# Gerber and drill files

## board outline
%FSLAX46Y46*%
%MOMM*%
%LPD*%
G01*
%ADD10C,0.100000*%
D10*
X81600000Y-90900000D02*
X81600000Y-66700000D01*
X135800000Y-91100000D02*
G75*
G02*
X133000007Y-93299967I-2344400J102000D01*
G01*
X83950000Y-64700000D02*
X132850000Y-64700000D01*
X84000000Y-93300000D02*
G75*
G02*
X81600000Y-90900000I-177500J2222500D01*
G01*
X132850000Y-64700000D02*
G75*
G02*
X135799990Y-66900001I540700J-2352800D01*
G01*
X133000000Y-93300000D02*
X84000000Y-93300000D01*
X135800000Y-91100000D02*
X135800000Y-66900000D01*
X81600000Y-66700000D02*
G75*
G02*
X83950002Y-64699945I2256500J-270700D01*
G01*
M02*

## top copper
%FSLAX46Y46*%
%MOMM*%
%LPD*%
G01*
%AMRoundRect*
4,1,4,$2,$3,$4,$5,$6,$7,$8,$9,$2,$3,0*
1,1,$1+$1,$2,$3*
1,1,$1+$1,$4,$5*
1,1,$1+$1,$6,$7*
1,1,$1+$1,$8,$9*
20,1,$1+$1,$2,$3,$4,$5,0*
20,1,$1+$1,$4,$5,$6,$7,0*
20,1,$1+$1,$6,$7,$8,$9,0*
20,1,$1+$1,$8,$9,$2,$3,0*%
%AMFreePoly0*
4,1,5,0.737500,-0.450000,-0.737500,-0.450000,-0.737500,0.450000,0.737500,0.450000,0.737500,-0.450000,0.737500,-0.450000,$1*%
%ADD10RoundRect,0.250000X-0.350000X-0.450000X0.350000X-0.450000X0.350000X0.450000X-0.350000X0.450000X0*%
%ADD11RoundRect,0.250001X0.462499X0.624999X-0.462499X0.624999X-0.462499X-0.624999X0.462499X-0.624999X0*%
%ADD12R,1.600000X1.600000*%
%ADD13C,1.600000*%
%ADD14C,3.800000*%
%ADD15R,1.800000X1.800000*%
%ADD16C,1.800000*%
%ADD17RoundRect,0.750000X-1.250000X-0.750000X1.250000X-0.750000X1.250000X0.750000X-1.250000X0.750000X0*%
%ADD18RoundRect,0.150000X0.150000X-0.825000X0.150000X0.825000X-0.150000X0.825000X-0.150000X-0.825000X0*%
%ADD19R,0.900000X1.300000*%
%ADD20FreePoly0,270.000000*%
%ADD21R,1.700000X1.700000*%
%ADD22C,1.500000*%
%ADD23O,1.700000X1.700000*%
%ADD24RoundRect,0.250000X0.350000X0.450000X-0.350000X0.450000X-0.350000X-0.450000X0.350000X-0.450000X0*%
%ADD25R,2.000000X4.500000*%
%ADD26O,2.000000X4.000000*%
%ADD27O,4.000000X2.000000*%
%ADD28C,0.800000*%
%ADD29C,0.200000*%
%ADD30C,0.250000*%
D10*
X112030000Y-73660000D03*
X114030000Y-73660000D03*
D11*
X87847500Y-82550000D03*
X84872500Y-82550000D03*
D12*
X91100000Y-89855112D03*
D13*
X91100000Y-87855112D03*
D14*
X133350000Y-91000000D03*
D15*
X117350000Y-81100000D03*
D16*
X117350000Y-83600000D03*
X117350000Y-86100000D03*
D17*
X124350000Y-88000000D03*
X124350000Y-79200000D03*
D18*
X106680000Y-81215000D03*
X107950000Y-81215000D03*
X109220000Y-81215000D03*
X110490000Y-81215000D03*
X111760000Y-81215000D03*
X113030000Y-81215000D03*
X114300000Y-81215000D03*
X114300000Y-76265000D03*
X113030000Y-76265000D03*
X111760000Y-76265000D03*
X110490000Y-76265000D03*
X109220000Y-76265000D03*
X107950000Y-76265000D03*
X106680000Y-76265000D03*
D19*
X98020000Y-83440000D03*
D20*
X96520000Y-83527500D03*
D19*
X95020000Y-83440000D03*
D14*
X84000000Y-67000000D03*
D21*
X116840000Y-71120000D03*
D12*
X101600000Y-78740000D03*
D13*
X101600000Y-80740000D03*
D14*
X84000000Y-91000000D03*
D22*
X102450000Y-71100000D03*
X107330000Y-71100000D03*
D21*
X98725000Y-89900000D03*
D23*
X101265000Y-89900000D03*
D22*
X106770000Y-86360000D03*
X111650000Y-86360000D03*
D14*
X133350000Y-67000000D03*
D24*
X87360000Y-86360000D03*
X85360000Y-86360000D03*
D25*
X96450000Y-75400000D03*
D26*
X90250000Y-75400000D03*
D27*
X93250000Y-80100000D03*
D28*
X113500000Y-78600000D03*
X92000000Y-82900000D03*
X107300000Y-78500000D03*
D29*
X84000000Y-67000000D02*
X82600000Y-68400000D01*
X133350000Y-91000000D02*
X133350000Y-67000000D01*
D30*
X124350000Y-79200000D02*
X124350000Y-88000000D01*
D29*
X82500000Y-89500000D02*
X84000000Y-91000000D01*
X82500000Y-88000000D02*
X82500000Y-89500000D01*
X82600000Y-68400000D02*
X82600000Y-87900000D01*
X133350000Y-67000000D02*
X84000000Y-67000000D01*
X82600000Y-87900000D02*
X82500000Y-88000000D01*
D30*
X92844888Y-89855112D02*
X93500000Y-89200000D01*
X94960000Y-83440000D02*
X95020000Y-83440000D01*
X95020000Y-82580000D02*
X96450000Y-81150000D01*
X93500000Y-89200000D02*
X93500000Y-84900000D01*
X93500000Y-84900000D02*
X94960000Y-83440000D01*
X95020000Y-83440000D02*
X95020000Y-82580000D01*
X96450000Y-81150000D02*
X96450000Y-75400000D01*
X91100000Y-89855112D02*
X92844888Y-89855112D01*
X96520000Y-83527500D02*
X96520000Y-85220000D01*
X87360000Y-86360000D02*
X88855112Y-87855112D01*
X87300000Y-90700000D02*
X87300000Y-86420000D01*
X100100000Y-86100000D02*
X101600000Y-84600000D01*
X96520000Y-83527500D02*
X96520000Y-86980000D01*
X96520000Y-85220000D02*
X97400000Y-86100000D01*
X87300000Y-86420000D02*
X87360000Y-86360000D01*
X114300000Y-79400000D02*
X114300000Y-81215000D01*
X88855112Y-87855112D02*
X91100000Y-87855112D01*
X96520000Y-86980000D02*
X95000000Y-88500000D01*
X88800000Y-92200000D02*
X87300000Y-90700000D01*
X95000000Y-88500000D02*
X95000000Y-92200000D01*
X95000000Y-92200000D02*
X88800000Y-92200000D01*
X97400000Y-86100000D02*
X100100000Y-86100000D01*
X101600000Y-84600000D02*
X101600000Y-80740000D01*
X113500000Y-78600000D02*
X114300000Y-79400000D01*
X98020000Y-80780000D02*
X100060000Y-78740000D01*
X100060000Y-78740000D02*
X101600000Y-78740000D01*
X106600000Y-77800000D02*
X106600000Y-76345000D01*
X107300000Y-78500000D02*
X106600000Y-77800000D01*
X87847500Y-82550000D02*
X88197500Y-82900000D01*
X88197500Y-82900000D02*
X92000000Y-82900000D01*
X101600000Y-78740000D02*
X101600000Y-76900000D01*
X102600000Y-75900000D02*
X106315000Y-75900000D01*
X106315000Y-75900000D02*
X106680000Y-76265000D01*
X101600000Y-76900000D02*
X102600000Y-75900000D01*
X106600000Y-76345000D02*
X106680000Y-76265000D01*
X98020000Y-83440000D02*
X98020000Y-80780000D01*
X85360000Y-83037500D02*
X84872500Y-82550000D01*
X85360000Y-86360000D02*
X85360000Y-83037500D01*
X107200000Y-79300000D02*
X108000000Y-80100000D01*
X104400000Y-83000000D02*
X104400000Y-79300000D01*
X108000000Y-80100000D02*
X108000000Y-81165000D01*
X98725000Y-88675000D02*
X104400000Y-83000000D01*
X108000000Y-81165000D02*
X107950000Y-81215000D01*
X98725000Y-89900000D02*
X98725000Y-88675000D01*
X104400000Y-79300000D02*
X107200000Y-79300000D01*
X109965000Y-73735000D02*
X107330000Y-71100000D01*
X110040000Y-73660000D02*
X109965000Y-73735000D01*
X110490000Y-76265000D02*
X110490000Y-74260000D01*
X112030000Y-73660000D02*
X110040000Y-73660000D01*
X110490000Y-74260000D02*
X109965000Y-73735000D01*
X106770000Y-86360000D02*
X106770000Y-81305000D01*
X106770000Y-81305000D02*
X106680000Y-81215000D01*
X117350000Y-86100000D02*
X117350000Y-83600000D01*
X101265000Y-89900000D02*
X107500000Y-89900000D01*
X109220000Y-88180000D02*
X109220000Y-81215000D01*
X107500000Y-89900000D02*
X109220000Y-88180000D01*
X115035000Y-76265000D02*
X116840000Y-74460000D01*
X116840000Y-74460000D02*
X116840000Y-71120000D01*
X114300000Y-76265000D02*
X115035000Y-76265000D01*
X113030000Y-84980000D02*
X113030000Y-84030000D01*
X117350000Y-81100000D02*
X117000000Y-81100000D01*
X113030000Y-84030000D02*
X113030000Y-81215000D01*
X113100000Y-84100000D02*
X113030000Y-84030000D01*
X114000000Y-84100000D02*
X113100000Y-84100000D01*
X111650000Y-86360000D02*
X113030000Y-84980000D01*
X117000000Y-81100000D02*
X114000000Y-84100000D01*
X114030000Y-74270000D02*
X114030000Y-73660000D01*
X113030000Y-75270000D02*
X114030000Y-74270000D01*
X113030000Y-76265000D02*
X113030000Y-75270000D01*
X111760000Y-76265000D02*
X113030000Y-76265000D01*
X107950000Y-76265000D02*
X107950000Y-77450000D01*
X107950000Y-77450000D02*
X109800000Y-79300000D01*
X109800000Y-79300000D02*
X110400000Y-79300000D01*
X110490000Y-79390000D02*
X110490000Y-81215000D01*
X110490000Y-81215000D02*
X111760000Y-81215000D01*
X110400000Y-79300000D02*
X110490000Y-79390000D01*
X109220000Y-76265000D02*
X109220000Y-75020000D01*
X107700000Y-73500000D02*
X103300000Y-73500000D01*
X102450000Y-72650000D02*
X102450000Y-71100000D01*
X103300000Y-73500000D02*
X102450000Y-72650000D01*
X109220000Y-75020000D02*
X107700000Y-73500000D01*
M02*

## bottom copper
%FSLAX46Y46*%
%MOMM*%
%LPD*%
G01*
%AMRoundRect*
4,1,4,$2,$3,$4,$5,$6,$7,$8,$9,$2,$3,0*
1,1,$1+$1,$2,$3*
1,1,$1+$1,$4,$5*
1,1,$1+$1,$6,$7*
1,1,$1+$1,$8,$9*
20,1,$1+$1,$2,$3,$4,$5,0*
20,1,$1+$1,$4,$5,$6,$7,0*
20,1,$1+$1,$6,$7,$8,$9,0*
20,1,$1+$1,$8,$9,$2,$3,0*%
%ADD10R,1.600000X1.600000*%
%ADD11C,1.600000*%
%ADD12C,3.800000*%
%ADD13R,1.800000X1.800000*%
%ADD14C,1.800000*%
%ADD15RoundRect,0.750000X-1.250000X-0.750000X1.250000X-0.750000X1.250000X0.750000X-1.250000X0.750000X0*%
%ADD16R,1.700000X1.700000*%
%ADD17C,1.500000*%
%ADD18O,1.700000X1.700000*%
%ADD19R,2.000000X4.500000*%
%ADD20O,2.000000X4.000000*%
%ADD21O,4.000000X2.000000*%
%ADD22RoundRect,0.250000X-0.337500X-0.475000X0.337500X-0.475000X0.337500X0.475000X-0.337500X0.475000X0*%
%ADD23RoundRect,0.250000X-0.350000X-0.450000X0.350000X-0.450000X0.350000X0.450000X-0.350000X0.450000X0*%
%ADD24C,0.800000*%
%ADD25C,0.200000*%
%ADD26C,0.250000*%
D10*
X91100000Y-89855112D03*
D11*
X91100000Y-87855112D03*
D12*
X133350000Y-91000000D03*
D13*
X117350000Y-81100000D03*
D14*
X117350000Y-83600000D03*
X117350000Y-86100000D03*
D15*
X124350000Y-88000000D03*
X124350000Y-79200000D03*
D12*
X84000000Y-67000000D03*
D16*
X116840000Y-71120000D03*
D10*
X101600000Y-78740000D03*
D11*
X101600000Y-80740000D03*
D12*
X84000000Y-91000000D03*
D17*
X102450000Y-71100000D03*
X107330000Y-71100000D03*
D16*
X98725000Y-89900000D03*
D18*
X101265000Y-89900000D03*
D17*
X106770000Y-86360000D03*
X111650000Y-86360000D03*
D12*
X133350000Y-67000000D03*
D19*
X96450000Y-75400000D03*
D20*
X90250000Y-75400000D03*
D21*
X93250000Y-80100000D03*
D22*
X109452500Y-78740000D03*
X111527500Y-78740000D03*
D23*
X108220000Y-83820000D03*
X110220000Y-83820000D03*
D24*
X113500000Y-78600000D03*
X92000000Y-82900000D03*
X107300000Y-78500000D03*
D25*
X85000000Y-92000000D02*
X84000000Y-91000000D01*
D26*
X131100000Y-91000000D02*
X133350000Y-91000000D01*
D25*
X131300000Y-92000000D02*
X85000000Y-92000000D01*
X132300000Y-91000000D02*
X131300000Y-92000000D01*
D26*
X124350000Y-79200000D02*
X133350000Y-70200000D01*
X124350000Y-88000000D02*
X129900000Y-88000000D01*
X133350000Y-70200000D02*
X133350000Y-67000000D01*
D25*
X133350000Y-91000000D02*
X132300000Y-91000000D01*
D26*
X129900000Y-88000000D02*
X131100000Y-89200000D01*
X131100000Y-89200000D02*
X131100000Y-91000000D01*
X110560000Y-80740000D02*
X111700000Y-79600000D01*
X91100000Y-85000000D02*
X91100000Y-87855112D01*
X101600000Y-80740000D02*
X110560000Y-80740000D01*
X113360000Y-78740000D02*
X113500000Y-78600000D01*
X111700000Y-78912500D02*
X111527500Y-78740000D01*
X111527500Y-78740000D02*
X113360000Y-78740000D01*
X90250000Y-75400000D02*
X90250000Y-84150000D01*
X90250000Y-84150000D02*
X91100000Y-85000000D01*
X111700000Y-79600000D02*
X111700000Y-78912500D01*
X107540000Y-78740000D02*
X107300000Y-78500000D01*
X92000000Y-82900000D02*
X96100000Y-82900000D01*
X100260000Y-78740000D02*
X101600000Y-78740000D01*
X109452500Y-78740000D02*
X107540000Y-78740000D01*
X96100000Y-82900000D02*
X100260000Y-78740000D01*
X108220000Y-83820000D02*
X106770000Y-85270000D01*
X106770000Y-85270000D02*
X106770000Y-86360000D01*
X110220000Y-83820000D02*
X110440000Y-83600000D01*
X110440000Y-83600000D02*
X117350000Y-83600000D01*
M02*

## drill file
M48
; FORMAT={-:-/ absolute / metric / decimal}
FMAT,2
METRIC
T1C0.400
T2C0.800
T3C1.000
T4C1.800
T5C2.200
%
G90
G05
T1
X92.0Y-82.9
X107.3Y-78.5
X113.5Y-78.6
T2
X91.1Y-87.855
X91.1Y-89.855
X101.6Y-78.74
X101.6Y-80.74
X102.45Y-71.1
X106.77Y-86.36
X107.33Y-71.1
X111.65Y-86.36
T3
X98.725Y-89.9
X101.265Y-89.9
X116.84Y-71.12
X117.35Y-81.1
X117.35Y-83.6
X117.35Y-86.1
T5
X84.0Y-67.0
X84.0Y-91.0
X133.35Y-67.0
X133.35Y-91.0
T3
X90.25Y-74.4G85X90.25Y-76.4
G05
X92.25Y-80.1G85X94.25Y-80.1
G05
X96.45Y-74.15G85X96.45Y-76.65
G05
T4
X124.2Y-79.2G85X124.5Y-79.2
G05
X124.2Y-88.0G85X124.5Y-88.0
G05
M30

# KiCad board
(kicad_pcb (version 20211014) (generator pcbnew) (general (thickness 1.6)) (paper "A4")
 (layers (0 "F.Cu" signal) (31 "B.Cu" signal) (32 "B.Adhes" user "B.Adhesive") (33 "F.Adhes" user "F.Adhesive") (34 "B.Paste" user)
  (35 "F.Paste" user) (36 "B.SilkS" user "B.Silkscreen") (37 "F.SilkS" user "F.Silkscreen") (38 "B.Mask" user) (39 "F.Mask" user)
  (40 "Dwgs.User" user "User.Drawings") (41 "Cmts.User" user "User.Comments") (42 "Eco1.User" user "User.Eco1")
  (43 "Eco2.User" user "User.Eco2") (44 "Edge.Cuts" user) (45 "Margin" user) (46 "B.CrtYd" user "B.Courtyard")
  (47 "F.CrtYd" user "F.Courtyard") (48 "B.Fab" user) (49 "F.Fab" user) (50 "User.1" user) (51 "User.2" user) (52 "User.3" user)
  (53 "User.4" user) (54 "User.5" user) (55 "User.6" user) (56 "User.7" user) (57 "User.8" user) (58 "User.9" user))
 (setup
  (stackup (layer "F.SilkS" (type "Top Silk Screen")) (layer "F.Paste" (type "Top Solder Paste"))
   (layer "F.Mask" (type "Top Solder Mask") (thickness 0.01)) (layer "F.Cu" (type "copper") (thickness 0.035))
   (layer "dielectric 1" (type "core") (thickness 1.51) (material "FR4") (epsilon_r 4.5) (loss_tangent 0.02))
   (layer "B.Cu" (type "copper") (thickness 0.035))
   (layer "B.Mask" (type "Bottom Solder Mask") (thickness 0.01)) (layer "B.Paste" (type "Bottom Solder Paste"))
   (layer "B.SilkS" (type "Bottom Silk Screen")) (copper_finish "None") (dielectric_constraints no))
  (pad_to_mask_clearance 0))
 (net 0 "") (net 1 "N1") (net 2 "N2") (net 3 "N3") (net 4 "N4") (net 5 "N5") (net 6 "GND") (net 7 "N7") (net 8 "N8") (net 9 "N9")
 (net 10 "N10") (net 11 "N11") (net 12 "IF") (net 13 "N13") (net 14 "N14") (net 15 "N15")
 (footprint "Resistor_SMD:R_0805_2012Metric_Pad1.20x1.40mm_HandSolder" (layer "F.Cu") (at 113.03 73.66)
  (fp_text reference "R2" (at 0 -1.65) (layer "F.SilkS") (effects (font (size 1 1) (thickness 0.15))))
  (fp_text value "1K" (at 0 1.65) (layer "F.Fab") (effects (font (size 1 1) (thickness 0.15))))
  (pad "1" smd roundrect (at -1 0) (size 1.2 1.4) (layers "F.Cu" "F.Paste" "F.Mask") (roundrect_rratio 0.208333) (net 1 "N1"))
  (pad "2" smd roundrect (at 1 0) (size 1.2 1.4) (layers "F.Cu" "F.Paste" "F.Mask") (roundrect_rratio 0.208333) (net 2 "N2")))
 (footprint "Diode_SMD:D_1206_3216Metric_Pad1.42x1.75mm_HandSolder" (layer "F.Cu") (at 86.36 82.55 180)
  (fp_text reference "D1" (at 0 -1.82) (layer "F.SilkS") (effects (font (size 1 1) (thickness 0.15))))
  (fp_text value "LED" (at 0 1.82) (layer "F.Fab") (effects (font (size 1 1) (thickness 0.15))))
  (pad "1" smd roundrect (at -1.4875 0 180) (size 1.425 1.75) (layers "F.Cu" "F.Paste" "F.Mask") (roundrect_rratio 0.175439) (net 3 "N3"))
  (pad "2" smd roundrect (at 1.4875 0 180) (size 1.425 1.75) (layers "F.Cu" "F.Paste" "F.Mask") (roundrect_rratio 0.175439) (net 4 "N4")))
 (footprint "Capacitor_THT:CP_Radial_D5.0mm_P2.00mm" (layer "F.Cu") (at 91.1 89.855112 90)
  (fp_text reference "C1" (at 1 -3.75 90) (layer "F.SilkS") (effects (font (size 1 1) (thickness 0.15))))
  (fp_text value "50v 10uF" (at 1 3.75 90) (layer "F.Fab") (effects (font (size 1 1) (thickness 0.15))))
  (pad "1" thru_hole rect (at 0 0 90) (size 1.6 1.6) (drill 0.8) (layers *.Cu *.Mask) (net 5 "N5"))
  (pad "2" thru_hole circle (at 2 0 90) (size 1.6 1.6) (drill 0.8) (layers *.Cu *.Mask) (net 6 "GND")))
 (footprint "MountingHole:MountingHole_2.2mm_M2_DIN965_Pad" (layer "F.Cu") (at 133.35 91)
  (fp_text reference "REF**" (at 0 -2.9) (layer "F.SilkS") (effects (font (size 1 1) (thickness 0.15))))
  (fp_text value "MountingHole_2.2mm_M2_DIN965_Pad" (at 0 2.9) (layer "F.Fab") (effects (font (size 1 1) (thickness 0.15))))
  (pad "1" thru_hole circle (at 0 0) (size 3.8 3.8) (drill 2.2) (layers F&B.Cu *.Mask)))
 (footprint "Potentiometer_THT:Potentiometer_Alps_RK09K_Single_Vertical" (layer "F.Cu") (at 117.35 81.1)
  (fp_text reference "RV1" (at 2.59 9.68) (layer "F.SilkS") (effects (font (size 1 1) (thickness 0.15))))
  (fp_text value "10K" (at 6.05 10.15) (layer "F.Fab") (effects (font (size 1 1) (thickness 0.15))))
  (pad "1" thru_hole rect (at 0 0) (size 1.8 1.8) (drill 1) (layers *.Cu *.Mask) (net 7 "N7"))
  (pad "2" thru_hole circle (at 0 2.5) (size 1.8 1.8) (drill 1) (layers *.Cu *.Mask) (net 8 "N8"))
  (pad "3" thru_hole circle (at 0 5) (size 1.8 1.8) (drill 1) (layers *.Cu *.Mask) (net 8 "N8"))
  (pad "MP" thru_hole roundrect (at 7 6.9) (size 4 3) (drill oval 2.1 1.8) (layers *.Cu *.Mask) (roundrect_rratio 0.25))
  (pad "MP" thru_hole roundrect (at 7 -1.9) (size 4 3) (drill oval 2.1 1.8) (layers *.Cu *.Mask) (roundrect_rratio 0.25)))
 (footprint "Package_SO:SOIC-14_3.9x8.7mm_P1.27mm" (layer "F.Cu") (at 110.49 78.74 90)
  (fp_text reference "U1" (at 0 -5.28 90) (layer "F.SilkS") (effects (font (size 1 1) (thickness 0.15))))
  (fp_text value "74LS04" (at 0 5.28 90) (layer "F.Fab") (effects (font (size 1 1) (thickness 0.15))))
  (pad "1" smd roundrect (at -2.475 -3.81 90) (size 1.95 0.6) (layers "F.Cu" "F.Paste" "F.Mask") (roundrect_rratio 0.25) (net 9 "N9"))
  (pad "2" smd roundrect (at -2.475 -2.54 90) (size 1.95 0.6) (layers "F.Cu" "F.Paste" "F.Mask") (roundrect_rratio 0.25) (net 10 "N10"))
  (pad "3" smd roundrect (at -2.475 -1.27 90) (size 1.95 0.6) (layers "F.Cu" "F.Paste" "F.Mask") (roundrect_rratio 0.25) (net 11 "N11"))
  (pad "4" smd roundrect (at -2.475 0 90) (size 1.95 0.6) (layers "F.Cu" "F.Paste" "F.Mask") (roundrect_rratio 0.25) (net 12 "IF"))
  (pad "5" smd roundrect (at -2.475 1.27 90) (size 1.95 0.6) (layers "F.Cu" "F.Paste" "F.Mask") (roundrect_rratio 0.25) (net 12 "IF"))
  (pad "6" smd roundrect (at -2.475 2.54 90) (size 1.95 0.6) (layers "F.Cu" "F.Paste" "F.Mask") (roundrect_rratio 0.25) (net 7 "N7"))
  (pad "7" smd roundrect (at -2.475 3.81 90) (size 1.95 0.6) (layers "F.Cu" "F.Paste" "F.Mask") (roundrect_rratio 0.25) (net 6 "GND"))
  (pad "8" smd roundrect (at 2.475 3.81 90) (size 1.95 0.6) (layers "F.Cu" "F.Paste" "F.Mask") (roundrect_rratio 0.25) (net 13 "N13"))
  (pad "9" smd roundrect (at 2.475 2.54 90) (size 1.95 0.6) (layers "F.Cu" "F.Paste" "F.Mask") (roundrect_rratio 0.25) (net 2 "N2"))
  (pad "10" smd roundrect (at 2.475 1.27 90) (size 1.95 0.6) (layers "F.Cu" "F.Paste" "F.Mask") (roundrect_rratio 0.25) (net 2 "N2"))
  (pad "11" smd roundrect (at 2.475 0 90) (size 1.95 0.6) (layers "F.Cu" "F.Paste" "F.Mask") (roundrect_rratio 0.25) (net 1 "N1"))
  (pad "12" smd roundrect (at 2.475 -1.27 90) (size 1.95 0.6) (layers "F.Cu" "F.Paste" "F.Mask") (roundrect_rratio 0.25) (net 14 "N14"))
  (pad "13" smd roundrect (at 2.475 -2.54 90) (size 1.95 0.6) (layers "F.Cu" "F.Paste" "F.Mask") (roundrect_rratio 0.25) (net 12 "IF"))
  (pad "14" smd roundrect (at 2.475 -3.81 90) (size 1.95 0.6) (layers "F.Cu" "F.Paste" "F.Mask") (roundrect_rratio 0.25) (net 3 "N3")))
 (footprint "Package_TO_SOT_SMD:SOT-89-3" (layer "F.Cu") (at 96.52 85.09 -90)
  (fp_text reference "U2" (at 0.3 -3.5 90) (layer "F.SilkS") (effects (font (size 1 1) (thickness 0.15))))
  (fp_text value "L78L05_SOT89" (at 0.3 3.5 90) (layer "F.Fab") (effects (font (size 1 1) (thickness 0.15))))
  (pad "1" smd rect (at -1.65 -1.5 270) (size 1.3 0.9) (layers "F.Cu" "F.Paste" "F.Mask") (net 3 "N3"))
  (pad "2" smd custom (at -1.5625 0 270) (size 1.475 0.9) (layers "F.Cu" "F.Paste" "F.Mask") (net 6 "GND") (zone_connect 2)
   (options (clearance outline) (anchor rect)) (primitives))
  (pad "3" smd rect (at -1.65 1.5 270) (size 1.3 0.9) (layers "F.Cu" "F.Paste" "F.Mask") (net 5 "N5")))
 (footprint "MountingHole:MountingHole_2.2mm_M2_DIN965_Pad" (layer "F.Cu") (at 84 67)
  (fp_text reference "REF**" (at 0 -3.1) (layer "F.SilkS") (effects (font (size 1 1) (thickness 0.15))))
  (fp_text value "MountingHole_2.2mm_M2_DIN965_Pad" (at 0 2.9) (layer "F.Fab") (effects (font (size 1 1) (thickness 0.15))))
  (pad "1" thru_hole circle (at 0 0) (size 3.8 3.8) (drill 2.2) (layers *.Cu *.Mask)))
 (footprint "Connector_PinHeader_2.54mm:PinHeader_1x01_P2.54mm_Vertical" (layer "F.Cu") (at 116.84 71.12)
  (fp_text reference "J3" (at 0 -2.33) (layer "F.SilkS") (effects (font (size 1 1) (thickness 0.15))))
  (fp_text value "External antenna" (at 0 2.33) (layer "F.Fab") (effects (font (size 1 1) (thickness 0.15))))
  (pad "1" thru_hole rect (at 0 0) (size 1.7 1.7) (drill 1) (layers *.Cu *.Mask) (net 13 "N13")))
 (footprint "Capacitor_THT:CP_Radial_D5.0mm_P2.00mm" (layer "F.Cu") (at 101.6 78.74 -90)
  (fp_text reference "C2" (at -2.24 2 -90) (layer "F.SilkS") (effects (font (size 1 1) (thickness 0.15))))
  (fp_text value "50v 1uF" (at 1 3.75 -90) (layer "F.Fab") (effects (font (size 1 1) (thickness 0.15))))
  (pad "1" thru_hole rect (at 0 0 270) (size 1.6 1.6) (drill 0.8) (layers *.Cu *.Mask) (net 3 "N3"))
  (pad "2" thru_hole circle (at 2 0 270) (size 1.6 1.6) (drill 0.8) (layers *.Cu *.Mask) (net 6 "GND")))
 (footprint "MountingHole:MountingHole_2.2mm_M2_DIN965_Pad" (layer "F.Cu") (at 84 91)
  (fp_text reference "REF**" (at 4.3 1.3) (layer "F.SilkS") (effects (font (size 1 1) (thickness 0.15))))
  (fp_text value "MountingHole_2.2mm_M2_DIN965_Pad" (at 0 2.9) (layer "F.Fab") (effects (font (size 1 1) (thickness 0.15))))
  (pad "1" thru_hole circle (at 0 0) (size 3.8 3.8) (drill 2.2) (layers *.Cu *.Mask)))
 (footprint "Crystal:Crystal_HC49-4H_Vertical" (layer "F.Cu") (at 102.45 71.1)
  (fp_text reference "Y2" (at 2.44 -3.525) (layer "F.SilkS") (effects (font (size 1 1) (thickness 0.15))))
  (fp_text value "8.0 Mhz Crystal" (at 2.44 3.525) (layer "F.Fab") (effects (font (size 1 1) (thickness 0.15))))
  (pad "1" thru_hole circle (at 0 0) (size 1.5 1.5) (drill 0.8) (layers *.Cu *.Mask) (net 14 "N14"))
  (pad "2" thru_hole circle (at 4.88 0) (size 1.5 1.5) (drill 0.8) (layers *.Cu *.Mask) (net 1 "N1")))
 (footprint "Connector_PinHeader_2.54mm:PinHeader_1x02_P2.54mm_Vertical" (layer "F.Cu") (at 98.725 89.9 90)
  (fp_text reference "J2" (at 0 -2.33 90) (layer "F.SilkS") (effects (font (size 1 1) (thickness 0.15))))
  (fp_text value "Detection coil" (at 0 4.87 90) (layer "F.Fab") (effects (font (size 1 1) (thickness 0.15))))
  (pad "1" thru_hole rect (at 0 0 90) (size 1.7 1.7) (drill 1) (layers *.Cu *.Mask) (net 10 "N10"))
  (pad "2" thru_hole oval (at 0 2.54 90) (size 1.7 1.7) (drill 1) (layers *.Cu *.Mask) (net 11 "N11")))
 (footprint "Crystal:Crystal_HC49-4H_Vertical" (layer "F.Cu") (at 106.77 86.36)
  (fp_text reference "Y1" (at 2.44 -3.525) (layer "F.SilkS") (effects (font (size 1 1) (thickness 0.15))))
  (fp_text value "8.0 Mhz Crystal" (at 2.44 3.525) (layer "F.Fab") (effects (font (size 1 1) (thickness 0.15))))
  (pad "1" thru_hole circle (at 0 0) (size 1.5 1.5) (drill 0.8) (layers *.Cu *.Mask) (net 9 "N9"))
  (pad "2" thru_hole circle (at 4.88 0) (size 1.5 1.5) (drill 0.8) (layers *.Cu *.Mask) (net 7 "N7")))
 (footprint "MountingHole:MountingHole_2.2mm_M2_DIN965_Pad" (layer "F.Cu") (at 133.35 67)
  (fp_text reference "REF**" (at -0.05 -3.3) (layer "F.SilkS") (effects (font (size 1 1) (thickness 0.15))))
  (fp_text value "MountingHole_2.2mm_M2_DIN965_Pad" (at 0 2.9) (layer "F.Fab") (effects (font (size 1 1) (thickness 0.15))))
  (pad "1" thru_hole circle (at 0 0) (size 3.8 3.8) (drill 2.2) (layers *.Cu *.Mask)))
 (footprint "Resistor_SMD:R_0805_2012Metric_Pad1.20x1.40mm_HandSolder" (layer "F.Cu") (at 86.36 86.36 180)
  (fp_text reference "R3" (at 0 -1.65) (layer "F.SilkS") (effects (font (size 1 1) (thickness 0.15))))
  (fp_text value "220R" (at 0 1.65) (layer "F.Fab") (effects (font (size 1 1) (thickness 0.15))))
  (pad "1" smd roundrect (at -1 0 180) (size 1.2 1.4) (layers "F.Cu" "F.Paste" "F.Mask") (roundrect_rratio 0.208333) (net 6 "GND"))
  (pad "2" smd roundrect (at 1 0 180) (size 1.2 1.4) (layers "F.Cu" "F.Paste" "F.Mask") (roundrect_rratio 0.208333) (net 4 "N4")))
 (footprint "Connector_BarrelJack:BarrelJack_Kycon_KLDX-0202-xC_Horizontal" (layer "F.Cu") (at 96.45 75.4)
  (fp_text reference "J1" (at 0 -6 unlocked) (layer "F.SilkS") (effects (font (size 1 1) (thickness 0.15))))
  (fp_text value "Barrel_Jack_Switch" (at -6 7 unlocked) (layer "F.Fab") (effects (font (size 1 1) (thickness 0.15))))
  (pad "1" thru_hole rect (at 0 0) (size 2 4.5) (drill oval 1 3.5) (layers *.Cu *.Mask) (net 5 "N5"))
  (pad "2" thru_hole oval (at -6.2 0) (size 2 4) (drill oval 1 3) (layers *.Cu *.Mask) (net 6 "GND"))
  (pad "3" thru_hole oval (at -3.2 4.7 90) (size 2 4) (drill oval 1 3) (layers *.Cu *.Mask) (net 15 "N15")))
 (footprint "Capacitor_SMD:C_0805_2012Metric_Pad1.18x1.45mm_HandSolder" (layer "B.Cu") (at 110.49 78.74)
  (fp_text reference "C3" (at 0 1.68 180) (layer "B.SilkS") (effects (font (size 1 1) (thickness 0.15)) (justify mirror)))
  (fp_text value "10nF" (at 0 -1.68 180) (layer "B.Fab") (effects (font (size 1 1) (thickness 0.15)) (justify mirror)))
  (pad "1" smd roundrect (at -1.0375 0) (size 1.175 1.45) (layers "B.Cu" "B.Paste" "B.Mask") (roundrect_rratio 0.212766) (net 3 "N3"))
  (pad "2" smd roundrect (at 1.0375 0) (size 1.175 1.45) (layers "B.Cu" "B.Paste" "B.Mask") (roundrect_rratio 0.212766) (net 6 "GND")))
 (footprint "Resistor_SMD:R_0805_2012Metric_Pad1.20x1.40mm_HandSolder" (layer "B.Cu") (at 109.22 83.82)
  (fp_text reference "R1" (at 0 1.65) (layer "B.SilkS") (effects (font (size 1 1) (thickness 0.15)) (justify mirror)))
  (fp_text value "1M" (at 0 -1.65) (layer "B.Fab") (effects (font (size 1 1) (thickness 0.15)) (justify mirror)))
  (pad "1" smd roundrect (at -1 0) (size 1.2 1.4) (layers "B.Cu" "B.Paste" "B.Mask") (roundrect_rratio 0.208333) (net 9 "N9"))
  (pad "2" smd roundrect (at 1 0) (size 1.2 1.4) (layers "B.Cu" "B.Paste" "B.Mask") (roundrect_rratio 0.208333) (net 8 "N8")))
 (gr_line (start 81.6 90.9) (end 81.6 66.7) (layer "Edge.Cuts") (width 0.1))
 (gr_arc (start 135.8 91.1) (mid 134.905392 92.843226) (end 133 93.3) (layer "Edge.Cuts") (width 0.1))
 (gr_line (start 83.95 64.7) (end 132.85 64.7) (layer "Edge.Cuts") (width 0.1))
 (gr_arc (start 84 93.3) (mid 82.24595 92.65405) (end 81.6 90.9) (layer "Edge.Cuts") (width 0.1))
 (gr_arc (start 132.85 64.7) (mid 134.833928 65.117573) (end 135.8 66.9) (layer "Edge.Cuts") (width 0.1))
 (gr_line (start 133 93.3) (end 84 93.3) (layer "Edge.Cuts") (width 0.1))
 (gr_line (start 135.8 91.1) (end 135.8 66.9) (layer "Edge.Cuts") (width 0.1))
 (gr_arc (start 81.6 66.7) (mid 82.383516 65.240007) (end 83.95 64.7) (layer "Edge.Cuts") (width 0.1))
 (segment (start 84 67) (end 82.6 68.4) (width 0.2) (layer "F.Cu") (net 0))
 (segment (start 133.35 91) (end 133.35 67) (width 0.2) (layer "F.Cu") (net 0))
 (segment (start 124.35 79.2) (end 124.35 88) (width 0.25) (layer "F.Cu") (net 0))
 (segment (start 82.5 89.5) (end 84 91) (width 0.2) (layer "F.Cu") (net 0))
 (segment (start 82.5 88) (end 82.5 89.5) (width 0.2) (layer "F.Cu") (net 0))
 (segment (start 82.6 68.4) (end 82.6 87.9) (width 0.2) (layer "F.Cu") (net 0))
 (segment (start 133.35 67) (end 84 67) (width 0.2) (layer "F.Cu") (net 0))
 (segment (start 82.6 87.9) (end 82.5 88) (width 0.2) (layer "F.Cu") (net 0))
 (segment (start 85 92) (end 84 91) (width 0.2) (layer "B.Cu") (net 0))
 (segment (start 131.1 91) (end 133.35 91) (width 0.25) (layer "B.Cu") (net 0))
 (segment (start 131.3 92) (end 85 92) (width 0.2) (layer "B.Cu") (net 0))
 (segment (start 132.3 91) (end 131.3 92) (width 0.2) (layer "B.Cu") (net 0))
 (segment (start 124.35 79.2) (end 133.35 70.2) (width 0.25) (layer "B.Cu") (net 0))
 (segment (start 124.35 88) (end 129.9 88) (width 0.25) (layer "B.Cu") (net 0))
 (segment (start 133.35 70.2) (end 133.35 67) (width 0.25) (layer "B.Cu") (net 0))
 (segment (start 133.35 91) (end 132.3 91) (width 0.2) (layer "B.Cu") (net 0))
 (segment (start 129.9 88) (end 131.1 89.2) (width 0.25) (layer "B.Cu") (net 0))
 (segment (start 131.1 89.2) (end 131.1 91) (width 0.25) (layer "B.Cu") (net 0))
 (segment (start 92.844888 89.855112) (end 93.5 89.2) (width 0.25) (layer "F.Cu") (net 5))
 (segment (start 94.96 83.44) (end 95.02 83.44) (width 0.25) (layer "F.Cu") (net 5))
 (segment (start 95.02 82.58) (end 96.45 81.15) (width 0.25) (layer "F.Cu") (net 5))
 (segment (start 93.5 89.2) (end 93.5 84.9) (width 0.25) (layer "F.Cu") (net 5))
 (segment (start 93.5 84.9) (end 94.96 83.44) (width 0.25) (layer "F.Cu") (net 5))
 (segment (start 95.02 83.44) (end 95.02 82.58) (width 0.25) (layer "F.Cu") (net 5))
 (segment (start 96.45 81.15) (end 96.45 75.4) (width 0.25) (layer "F.Cu") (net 5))
 (segment (start 91.1 89.855112) (end 92.844888 89.855112) (width 0.25) (layer "F.Cu") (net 5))
 (segment (start 96.52 83.5275) (end 96.52 85.22) (width 0.25) (layer "F.Cu") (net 6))
 (segment (start 87.36 86.36) (end 88.855112 87.855112) (width 0.25) (layer "F.Cu") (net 6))
 (segment (start 87.3 90.7) (end 87.3 86.42) (width 0.25) (layer "F.Cu") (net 6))
 (segment (start 100.1 86.1) (end 101.6 84.6) (width 0.25) (layer "F.Cu") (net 6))
 (segment (start 96.52 83.5275) (end 96.52 86.98) (width 0.25) (layer "F.Cu") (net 6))
 (segment (start 96.52 85.22) (end 97.4 86.1) (width 0.25) (layer "F.Cu") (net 6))
 (segment (start 87.3 86.42) (end 87.36 86.36) (width 0.25) (layer "F.Cu") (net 6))
 (segment (start 114.3 79.4) (end 114.3 81.215) (width 0.25) (layer "F.Cu") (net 6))
 (segment (start 88.855112 87.855112) (end 91.1 87.855112) (width 0.25) (layer "F.Cu") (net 6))
 (segment (start 96.52 86.98) (end 95 88.5) (width 0.25) (layer "F.Cu") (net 6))
 (segment (start 88.8 92.2) (end 87.3 90.7) (width 0.25) (layer "F.Cu") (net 6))
 (segment (start 95 88.5) (end 95 92.2) (width 0.25) (layer "F.Cu") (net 6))
 (segment (start 95 92.2) (end 88.8 92.2) (width 0.25) (layer "F.Cu") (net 6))
 (segment (start 97.4 86.1) (end 100.1 86.1) (width 0.25) (layer "F.Cu") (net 6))
 (segment (start 101.6 84.6) (end 101.6 80.74) (width 0.25) (layer "F.Cu") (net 6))
 (segment (start 113.5 78.6) (end 114.3 79.4) (width 0.25) (layer "F.Cu") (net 6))
 (via (at 113.5 78.6) (size 0.8) (drill 0.4) (layers "F.Cu" "B.Cu") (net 6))
 (segment (start 110.56 80.74) (end 111.7 79.6) (width 0.25) (layer "B.Cu") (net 6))
 (segment (start 91.1 85) (end 91.1 87.855112) (width 0.25) (layer "B.Cu") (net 6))
 (segment (start 101.6 80.74) (end 110.56 80.74) (width 0.25) (layer "B.Cu") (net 6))
 (segment (start 113.36 78.74) (end 113.5 78.6) (width 0.25) (layer "B.Cu") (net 6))
 (segment (start 111.7 78.9125) (end 111.5275 78.74) (width 0.25) (layer "B.Cu") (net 6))
 (segment (start 111.5275 78.74) (end 113.36 78.74) (width 0.25) (layer "B.Cu") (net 6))
 (segment (start 90.25 75.4) (end 90.25 84.15) (width 0.25) (layer "B.Cu") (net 6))
 (segment (start 90.25 84.15) (end 91.1 85) (width 0.25) (layer "B.Cu") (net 6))
 (segment (start 111.7 79.6) (end 111.7 78.9125) (width 0.25) (layer "B.Cu") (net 6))
 (segment (start 98.02 80.78) (end 100.06 78.74) (width 0.25) (layer "F.Cu") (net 3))
 (segment (start 100.06 78.74) (end 101.6 78.74) (width 0.25) (layer "F.Cu") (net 3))
 (segment (start 106.6 77.8) (end 106.6 76.345) (width 0.25) (layer "F.Cu") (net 3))
 (segment (start 107.3 78.5) (end 106.6 77.8) (width 0.25) (layer "F.Cu") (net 3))
 (segment (start 87.8475 82.55) (end 88.1975 82.9) (width 0.25) (layer "F.Cu") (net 3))
 (segment (start 88.1975 82.9) (end 92 82.9) (width 0.25) (layer "F.Cu") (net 3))
 (segment (start 101.6 78.74) (end 101.6 76.9) (width 0.25) (layer "F.Cu") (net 3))
 (segment (start 102.6 75.9) (end 106.315 75.9) (width 0.25) (layer "F.Cu") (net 3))
 (segment (start 106.315 75.9) (end 106.68 76.265) (width 0.25) (layer "F.Cu") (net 3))
 (segment (start 101.6 76.9) (end 102.6 75.9) (width 0.25) (layer "F.Cu") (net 3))
 (segment (start 106.6 76.345) (end 106.68 76.265) (width 0.25) (layer "F.Cu") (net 3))
 (segment (start 98.02 83.44) (end 98.02 80.78) (width 0.25) (layer "F.Cu") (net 3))
 (via (at 92 82.9) (size 0.8) (drill 0.4) (layers "F.Cu" "B.Cu") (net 3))
 (via (at 107.3 78.5) (size 0.8) (drill 0.4) (layers "F.Cu" "B.Cu") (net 3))
 (segment (start 107.54 78.74) (end 107.3 78.5) (width 0.25) (layer "B.Cu") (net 3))
 (segment (start 92 82.9) (end 96.1 82.9) (width 0.25) (layer "B.Cu") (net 3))
 (segment (start 100.26 78.74) (end 101.6 78.74) (width 0.25) (layer "B.Cu") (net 3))
 (segment (start 109.4525 78.74) (end 107.54 78.74) (width 0.25) (layer "B.Cu") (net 3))
 (segment (start 96.1 82.9) (end 100.26 78.74) (width 0.25) (layer "B.Cu") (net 3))
 (segment (start 85.36 83.0375) (end 84.8725 82.55) (width 0.25) (layer "F.Cu") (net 4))
 (segment (start 85.36 86.36) (end 85.36 83.0375) (width 0.25) (layer "F.Cu") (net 4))
 (segment (start 107.2 79.3) (end 108 80.1) (width 0.25) (layer "F.Cu") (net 10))
 (segment (start 104.4 83) (end 104.4 79.3) (width 0.25) (layer "F.Cu") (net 10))
 (segment (start 108 80.1) (end 108 81.165) (width 0.25) (layer "F.Cu") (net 10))
 (segment (start 98.725 88.675) (end 104.4 83) (width 0.25) (layer "F.Cu") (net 10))
 (segment (start 108 81.165) (end 107.95 81.215) (width 0.25) (layer "F.Cu") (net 10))
 (segment (start 98.725 89.9) (end 98.725 88.675) (width 0.25) (layer "F.Cu") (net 10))
 (segment (start 104.4 79.3) (end 107.2 79.3) (width 0.25) (layer "F.Cu") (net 10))
 (segment (start 109.965 73.735) (end 107.33 71.1) (width 0.25) (layer "F.Cu") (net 1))
 (segment (start 110.04 73.66) (end 109.965 73.735) (width 0.25) (layer "F.Cu") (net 1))
 (segment (start 110.49 76.265) (end 110.49 74.26) (width 0.25) (layer "F.Cu") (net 1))
 (segment (start 112.03 73.66) (end 110.04 73.66) (width 0.25) (layer "F.Cu") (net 1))
 (segment (start 110.49 74.26) (end 109.965 73.735) (width 0.25) (layer "F.Cu") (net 1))
 (segment (start 106.77 86.36) (end 106.77 81.305) (width 0.25) (layer "F.Cu") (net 9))
 (segment (start 106.77 81.305) (end 106.68 81.215) (width 0.25) (layer "F.Cu") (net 9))
 (segment (start 108.22 83.82) (end 106.77 85.27) (width 0.25) (layer "B.Cu") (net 9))
 (segment (start 106.77 85.27) (end 106.77 86.36) (width 0.25) (layer "B.Cu") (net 9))
 (segment (start 117.35 86.1) (end 117.35 83.6) (width 0.25) (layer "F.Cu") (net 8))
 (segment (start 110.22 83.82) (end 110.44 83.6) (width 0.25) (layer "B.Cu") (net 8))
 (segment (start 110.44 83.6) (end 117.35 83.6) (width 0.25) (layer "B.Cu") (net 8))
 (segment (start 101.265 89.9) (end 107.5 89.9) (width 0.25) (layer "F.Cu") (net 11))
 (segment (start 109.22 88.18) (end 109.22 81.215) (width 0.25) (layer "F.Cu") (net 11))
 (segment (start 107.5 89.9) (end 109.22 88.18) (width 0.25) (layer "F.Cu") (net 11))
 (segment (start 115.035 76.265) (end 116.84 74.46) (width 0.25) (layer "F.Cu") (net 13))
 (segment (start 116.84 74.46) (end 116.84 71.12) (width 0.25) (layer "F.Cu") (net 13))
 (segment (start 114.3 76.265) (end 115.035 76.265) (width 0.25) (layer "F.Cu") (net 13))
 (segment (start 113.03 84.98) (end 113.03 84.03) (width 0.25) (layer "F.Cu") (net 7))
 (segment (start 117.35 81.1) (end 117 81.1) (width 0.25) (layer "F.Cu") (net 7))
 (segment (start 113.03 84.03) (end 113.03 81.215) (width 0.25) (layer "F.Cu") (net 7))
 (segment (start 113.1 84.1) (end 113.03 84.03) (width 0.25) (layer "F.Cu") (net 7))
 (segment (start 114 84.1) (end 113.1 84.1) (width 0.25) (layer "F.Cu") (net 7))
 (segment (start 111.65 86.36) (end 113.03 84.98) (width 0.25) (layer "F.Cu") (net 7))
 (segment (start 117 81.1) (end 114 84.1) (width 0.25) (layer "F.Cu") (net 7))
 (segment (start 114.03 74.27) (end 114.03 73.66) (width 0.25) (layer "F.Cu") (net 2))
 (segment (start 113.03 75.27) (end 114.03 74.27) (width 0.25) (layer "F.Cu") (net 2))
 (segment (start 113.03 76.265) (end 113.03 75.27) (width 0.25) (layer "F.Cu") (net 2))
 (segment (start 111.76 76.265) (end 113.03 76.265) (width 0.25) (layer "F.Cu") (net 2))
 (segment (start 107.95 76.265) (end 107.95 77.45) (width 0.25) (layer "F.Cu") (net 12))
 (segment (start 107.95 77.45) (end 109.8 79.3) (width 0.25) (layer "F.Cu") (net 12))
 (segment (start 109.8 79.3) (end 110.4 79.3) (width 0.25) (layer "F.Cu") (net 12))
 (segment (start 110.49 79.39) (end 110.49 81.215) (width 0.25) (layer "F.Cu") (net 12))
 (segment (start 110.49 81.215) (end 111.76 81.215) (width 0.25) (layer "F.Cu") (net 12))
 (segment (start 110.4 79.3) (end 110.49 79.39) (width 0.25) (layer "F.Cu") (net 12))
 (segment (start 109.22 76.265) (end 109.22 75.02) (width 0.25) (layer "F.Cu") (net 14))
 (segment (start 107.7 73.5) (end 103.3 73.5) (width 0.25) (layer "F.Cu") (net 14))
 (segment (start 102.45 72.65) (end 102.45 71.1) (width 0.25) (layer "F.Cu") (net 14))
 (segment (start 103.3 73.5) (end 102.45 72.65) (width 0.25) (layer "F.Cu") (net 14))
 (segment (start 109.22 75.02) (end 107.7 73.5) (width 0.25) (layer "F.Cu") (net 14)))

